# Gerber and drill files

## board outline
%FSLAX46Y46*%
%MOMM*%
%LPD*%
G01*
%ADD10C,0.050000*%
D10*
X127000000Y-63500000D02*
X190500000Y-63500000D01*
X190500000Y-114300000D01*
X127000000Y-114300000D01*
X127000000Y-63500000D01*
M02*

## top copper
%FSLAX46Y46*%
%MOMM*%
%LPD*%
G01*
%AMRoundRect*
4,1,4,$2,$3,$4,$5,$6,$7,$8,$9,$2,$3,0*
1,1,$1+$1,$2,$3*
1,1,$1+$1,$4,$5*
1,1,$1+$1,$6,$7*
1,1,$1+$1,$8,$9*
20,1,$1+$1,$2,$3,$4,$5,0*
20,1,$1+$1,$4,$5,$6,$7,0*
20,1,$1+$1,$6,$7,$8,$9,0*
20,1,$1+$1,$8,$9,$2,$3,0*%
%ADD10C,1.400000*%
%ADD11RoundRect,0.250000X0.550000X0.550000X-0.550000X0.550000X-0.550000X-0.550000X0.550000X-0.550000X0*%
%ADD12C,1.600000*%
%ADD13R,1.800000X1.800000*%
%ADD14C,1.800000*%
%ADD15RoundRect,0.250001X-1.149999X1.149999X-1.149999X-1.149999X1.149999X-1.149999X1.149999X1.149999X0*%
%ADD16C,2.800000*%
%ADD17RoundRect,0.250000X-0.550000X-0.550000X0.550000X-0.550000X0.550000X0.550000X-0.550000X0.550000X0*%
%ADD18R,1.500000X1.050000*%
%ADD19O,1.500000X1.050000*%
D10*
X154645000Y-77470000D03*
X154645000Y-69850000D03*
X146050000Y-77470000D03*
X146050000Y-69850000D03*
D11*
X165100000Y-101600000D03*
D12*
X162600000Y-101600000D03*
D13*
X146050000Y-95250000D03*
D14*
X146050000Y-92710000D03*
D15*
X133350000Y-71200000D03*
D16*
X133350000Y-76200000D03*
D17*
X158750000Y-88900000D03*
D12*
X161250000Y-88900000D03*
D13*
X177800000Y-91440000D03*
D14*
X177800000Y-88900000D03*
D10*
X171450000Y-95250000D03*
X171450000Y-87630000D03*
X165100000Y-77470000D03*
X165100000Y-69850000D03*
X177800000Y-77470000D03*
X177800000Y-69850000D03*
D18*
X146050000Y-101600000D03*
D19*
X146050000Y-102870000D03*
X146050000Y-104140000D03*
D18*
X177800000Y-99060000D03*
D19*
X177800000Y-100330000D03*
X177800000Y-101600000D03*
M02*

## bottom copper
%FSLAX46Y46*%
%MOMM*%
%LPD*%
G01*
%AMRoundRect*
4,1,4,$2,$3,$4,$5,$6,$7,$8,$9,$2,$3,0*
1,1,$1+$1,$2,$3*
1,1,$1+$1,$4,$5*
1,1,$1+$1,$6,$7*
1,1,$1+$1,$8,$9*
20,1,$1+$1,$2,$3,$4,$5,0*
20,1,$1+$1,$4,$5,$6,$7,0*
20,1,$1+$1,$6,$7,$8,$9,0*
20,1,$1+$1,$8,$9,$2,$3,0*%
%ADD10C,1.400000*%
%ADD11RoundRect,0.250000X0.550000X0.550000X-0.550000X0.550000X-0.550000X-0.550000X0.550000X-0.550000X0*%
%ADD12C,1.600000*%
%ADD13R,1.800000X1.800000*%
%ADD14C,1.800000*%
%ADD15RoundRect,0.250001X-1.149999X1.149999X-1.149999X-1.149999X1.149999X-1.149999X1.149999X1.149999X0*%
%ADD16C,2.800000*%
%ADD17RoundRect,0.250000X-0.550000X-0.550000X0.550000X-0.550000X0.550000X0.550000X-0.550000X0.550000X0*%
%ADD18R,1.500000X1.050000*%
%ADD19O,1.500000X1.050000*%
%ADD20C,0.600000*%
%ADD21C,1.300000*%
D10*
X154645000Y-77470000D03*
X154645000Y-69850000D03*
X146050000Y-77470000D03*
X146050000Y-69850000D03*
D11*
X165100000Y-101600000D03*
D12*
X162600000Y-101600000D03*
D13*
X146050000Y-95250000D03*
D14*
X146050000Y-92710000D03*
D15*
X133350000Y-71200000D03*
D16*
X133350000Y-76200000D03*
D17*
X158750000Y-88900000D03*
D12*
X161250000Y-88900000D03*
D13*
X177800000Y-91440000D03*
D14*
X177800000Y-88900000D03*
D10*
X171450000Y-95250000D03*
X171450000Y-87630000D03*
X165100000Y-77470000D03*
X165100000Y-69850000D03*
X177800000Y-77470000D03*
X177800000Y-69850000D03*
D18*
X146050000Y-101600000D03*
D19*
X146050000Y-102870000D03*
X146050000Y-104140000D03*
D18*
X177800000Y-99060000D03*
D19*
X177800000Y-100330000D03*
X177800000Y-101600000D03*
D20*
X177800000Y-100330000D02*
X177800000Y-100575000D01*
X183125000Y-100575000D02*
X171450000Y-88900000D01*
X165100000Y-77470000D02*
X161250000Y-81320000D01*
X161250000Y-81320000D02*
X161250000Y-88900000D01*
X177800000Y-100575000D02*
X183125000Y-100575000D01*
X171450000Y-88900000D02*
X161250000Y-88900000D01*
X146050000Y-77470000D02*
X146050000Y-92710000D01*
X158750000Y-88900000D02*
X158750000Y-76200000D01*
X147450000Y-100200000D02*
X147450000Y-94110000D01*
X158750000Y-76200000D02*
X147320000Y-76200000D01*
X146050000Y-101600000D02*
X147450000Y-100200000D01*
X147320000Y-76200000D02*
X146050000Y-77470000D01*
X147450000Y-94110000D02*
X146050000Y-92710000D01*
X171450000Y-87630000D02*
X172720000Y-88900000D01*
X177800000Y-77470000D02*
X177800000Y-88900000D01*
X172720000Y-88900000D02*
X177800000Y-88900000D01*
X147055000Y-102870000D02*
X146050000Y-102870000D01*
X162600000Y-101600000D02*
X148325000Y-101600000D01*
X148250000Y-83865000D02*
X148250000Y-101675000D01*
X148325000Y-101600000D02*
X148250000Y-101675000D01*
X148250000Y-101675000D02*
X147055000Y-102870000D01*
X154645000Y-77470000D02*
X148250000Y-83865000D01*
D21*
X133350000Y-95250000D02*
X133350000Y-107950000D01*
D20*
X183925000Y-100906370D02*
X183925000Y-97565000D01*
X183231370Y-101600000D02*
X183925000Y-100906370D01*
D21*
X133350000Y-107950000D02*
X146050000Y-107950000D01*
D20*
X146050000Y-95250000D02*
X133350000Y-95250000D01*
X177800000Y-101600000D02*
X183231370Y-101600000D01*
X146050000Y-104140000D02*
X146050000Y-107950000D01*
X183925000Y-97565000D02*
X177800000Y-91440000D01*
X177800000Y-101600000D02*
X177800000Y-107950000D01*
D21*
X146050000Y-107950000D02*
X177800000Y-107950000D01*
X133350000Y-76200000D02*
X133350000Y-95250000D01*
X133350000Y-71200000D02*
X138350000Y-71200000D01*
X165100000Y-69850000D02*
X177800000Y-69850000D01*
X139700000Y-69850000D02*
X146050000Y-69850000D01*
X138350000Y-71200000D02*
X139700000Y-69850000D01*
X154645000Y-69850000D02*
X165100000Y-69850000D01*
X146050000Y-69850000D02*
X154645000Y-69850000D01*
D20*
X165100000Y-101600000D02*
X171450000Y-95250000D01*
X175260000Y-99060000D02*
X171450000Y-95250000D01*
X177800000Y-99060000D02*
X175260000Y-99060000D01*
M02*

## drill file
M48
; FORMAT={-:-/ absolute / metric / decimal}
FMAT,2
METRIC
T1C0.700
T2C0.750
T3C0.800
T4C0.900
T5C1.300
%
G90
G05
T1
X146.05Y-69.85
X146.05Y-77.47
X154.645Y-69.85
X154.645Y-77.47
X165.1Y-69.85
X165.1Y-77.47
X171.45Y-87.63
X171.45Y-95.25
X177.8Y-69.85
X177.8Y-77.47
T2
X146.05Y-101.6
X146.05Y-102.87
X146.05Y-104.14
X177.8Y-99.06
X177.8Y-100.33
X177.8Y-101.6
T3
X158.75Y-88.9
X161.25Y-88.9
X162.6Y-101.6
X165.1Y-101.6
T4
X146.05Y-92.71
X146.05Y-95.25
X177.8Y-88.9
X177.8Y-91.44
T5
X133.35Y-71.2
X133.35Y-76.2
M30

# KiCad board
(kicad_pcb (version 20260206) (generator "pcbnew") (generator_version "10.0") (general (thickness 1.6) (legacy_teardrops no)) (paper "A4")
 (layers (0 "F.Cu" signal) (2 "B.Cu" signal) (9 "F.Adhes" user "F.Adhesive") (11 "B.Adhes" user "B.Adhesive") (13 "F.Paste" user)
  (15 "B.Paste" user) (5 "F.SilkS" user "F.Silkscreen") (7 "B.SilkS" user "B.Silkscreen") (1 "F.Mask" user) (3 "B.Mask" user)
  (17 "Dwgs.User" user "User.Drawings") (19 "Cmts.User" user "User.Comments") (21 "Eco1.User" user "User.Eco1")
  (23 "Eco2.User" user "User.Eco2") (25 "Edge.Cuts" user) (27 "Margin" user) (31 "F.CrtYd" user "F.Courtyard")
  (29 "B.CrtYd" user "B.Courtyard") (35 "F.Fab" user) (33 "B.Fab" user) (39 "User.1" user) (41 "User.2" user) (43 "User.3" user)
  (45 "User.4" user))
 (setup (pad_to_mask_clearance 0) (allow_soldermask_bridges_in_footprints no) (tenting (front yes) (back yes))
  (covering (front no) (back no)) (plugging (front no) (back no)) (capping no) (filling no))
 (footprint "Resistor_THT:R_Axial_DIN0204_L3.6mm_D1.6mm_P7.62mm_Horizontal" (layer "F.Cu") (at 154.645 77.47 90)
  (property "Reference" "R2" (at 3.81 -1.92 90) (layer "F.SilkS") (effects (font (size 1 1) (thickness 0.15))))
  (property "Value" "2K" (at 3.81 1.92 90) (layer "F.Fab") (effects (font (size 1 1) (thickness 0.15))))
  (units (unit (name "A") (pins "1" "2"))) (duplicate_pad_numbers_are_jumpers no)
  (pad "1" thru_hole circle (at 0 0 90) (size 1.4 1.4) (drill 0.7) (layers "*.Cu" "*.Mask") (remove_unused_layers no) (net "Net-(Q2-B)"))
  (pad "2" thru_hole circle (at 7.62 0 90) (size 1.4 1.4) (drill 0.7) (layers "*.Cu" "*.Mask") (remove_unused_layers no) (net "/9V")))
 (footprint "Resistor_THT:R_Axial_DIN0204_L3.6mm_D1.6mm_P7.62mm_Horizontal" (layer "F.Cu") (at 146.05 77.47 90)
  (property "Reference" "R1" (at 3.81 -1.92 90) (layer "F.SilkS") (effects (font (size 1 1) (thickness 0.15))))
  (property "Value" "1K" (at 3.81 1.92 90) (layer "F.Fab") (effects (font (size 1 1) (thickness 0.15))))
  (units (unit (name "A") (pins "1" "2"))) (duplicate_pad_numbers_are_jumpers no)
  (pad "1" thru_hole circle (at 0 0 90) (size 1.4 1.4) (drill 0.7) (layers "*.Cu" "*.Mask") (remove_unused_layers no) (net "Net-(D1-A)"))
  (pad "2" thru_hole circle (at 7.62 0 90) (size 1.4 1.4) (drill 0.7) (layers "*.Cu" "*.Mask") (remove_unused_layers no) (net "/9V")))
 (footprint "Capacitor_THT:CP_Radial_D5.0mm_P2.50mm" (layer "F.Cu") (at 165.1 101.6 180)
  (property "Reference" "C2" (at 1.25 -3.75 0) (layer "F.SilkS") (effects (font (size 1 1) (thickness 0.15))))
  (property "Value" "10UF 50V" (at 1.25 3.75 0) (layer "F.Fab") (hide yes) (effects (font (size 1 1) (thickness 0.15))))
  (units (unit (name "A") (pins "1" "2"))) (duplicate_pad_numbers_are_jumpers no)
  (pad "1" thru_hole roundrect (at 0 0 180) (size 1.6 1.6) (drill 0.8) (layers "*.Cu" "*.Mask") (remove_unused_layers no)
   (roundrect_rratio 0.15625) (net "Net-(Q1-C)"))
  (pad "2" thru_hole circle (at 2.5 0 180) (size 1.6 1.6) (drill 0.8) (layers "*.Cu" "*.Mask") (remove_unused_layers no) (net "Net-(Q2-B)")))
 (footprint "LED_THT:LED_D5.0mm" (layer "F.Cu") (at 146.05 95.25 90)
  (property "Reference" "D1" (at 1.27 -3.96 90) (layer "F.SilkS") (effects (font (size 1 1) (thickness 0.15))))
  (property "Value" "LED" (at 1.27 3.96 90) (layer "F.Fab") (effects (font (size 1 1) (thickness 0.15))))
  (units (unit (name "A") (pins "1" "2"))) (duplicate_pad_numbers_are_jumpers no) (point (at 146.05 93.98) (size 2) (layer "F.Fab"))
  (pad "1" thru_hole rect (at 0 0 90) (size 1.8 1.8) (drill 0.9) (layers "*.Cu" "*.Mask") (remove_unused_layers no) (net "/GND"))
  (pad "2" thru_hole circle (at 2.54 0 90) (size 1.8 1.8) (drill 0.9) (layers "*.Cu" "*.Mask") (remove_unused_layers no) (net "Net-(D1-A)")))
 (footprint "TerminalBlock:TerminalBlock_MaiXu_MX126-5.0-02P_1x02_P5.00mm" (layer "F.Cu") (at 133.35 71.2 -90)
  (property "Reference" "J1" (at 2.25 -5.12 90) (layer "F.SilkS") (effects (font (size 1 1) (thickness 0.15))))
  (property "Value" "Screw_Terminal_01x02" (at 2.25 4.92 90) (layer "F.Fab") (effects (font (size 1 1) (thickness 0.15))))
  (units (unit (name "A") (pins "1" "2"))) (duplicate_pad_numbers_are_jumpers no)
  (pad "1" thru_hole roundrect (at 0 0 270) (size 2.8 2.8) (drill 1.3) (layers "*.Cu" "*.Mask") (remove_unused_layers no)
   (roundrect_rratio 0.089286) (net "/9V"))
  (pad "2" thru_hole circle (at 5 0 270) (size 2.8 2.8) (drill 1.3) (layers "*.Cu" "*.Mask") (remove_unused_layers no) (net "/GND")))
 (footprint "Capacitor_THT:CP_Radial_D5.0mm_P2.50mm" (layer "F.Cu") (at 158.75 88.9)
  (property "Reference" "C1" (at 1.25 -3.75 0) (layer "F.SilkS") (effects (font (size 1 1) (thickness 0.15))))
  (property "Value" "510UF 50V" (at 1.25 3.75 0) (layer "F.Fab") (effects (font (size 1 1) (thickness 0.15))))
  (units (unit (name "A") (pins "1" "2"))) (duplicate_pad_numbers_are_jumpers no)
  (pad "1" thru_hole roundrect (at 0 0) (size 1.6 1.6) (drill 0.8) (layers "*.Cu" "*.Mask") (remove_unused_layers no)
   (roundrect_rratio 0.15625) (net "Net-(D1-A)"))
  (pad "2" thru_hole circle (at 2.5 0) (size 1.6 1.6) (drill 0.8) (layers "*.Cu" "*.Mask") (remove_unused_layers no) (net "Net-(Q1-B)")))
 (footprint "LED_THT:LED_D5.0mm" (layer "F.Cu") (at 177.8 91.44 90)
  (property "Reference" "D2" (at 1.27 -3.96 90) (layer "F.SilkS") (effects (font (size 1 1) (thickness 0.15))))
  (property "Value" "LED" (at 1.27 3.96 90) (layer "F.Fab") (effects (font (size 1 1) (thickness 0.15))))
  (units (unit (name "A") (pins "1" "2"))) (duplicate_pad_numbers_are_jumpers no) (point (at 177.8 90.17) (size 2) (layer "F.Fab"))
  (pad "1" thru_hole rect (at 0 0 90) (size 1.8 1.8) (drill 0.9) (layers "*.Cu" "*.Mask") (remove_unused_layers no) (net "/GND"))
  (pad "2" thru_hole circle (at 2.54 0 90) (size 1.8 1.8) (drill 0.9) (layers "*.Cu" "*.Mask") (remove_unused_layers no) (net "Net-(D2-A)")))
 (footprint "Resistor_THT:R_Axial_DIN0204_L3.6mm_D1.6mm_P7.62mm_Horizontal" (layer "F.Cu") (at 171.45 95.25 90)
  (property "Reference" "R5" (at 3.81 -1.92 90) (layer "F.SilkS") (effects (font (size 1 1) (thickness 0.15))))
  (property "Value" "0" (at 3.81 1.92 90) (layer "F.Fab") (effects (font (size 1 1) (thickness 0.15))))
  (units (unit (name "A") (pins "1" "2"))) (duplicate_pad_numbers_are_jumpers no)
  (pad "1" thru_hole circle (at 0 0 90) (size 1.4 1.4) (drill 0.7) (layers "*.Cu" "*.Mask") (remove_unused_layers no) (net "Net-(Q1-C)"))
  (pad "2" thru_hole circle (at 7.62 0 90) (size 1.4 1.4) (drill 0.7) (layers "*.Cu" "*.Mask") (remove_unused_layers no) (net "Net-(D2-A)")))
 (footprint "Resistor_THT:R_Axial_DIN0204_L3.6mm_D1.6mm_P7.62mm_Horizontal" (layer "F.Cu") (at 165.1 77.47 90)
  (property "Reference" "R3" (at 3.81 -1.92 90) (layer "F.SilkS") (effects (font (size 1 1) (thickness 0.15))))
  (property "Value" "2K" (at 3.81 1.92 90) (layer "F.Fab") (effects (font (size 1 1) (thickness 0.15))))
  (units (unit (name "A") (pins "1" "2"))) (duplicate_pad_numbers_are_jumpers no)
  (pad "1" thru_hole circle (at 0 0 90) (size 1.4 1.4) (drill 0.7) (layers "*.Cu" "*.Mask") (remove_unused_layers no) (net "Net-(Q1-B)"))
  (pad "2" thru_hole circle (at 7.62 0 90) (size 1.4 1.4) (drill 0.7) (layers "*.Cu" "*.Mask") (remove_unused_layers no) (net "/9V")))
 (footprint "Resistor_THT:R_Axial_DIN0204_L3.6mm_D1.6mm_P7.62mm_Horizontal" (layer "F.Cu") (at 177.8 77.47 90)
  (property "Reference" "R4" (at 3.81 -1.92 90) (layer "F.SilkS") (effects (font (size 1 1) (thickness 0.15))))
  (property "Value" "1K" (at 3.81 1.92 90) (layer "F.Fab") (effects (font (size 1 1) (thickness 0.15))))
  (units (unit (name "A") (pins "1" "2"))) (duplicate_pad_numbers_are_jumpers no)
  (pad "1" thru_hole circle (at 0 0 90) (size 1.4 1.4) (drill 0.7) (layers "*.Cu" "*.Mask") (remove_unused_layers no) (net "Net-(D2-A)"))
  (pad "2" thru_hole circle (at 7.62 0 90) (size 1.4 1.4) (drill 0.7) (layers "*.Cu" "*.Mask") (remove_unused_layers no) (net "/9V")))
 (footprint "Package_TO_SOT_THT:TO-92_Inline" (layer "F.Cu") (at 146.05 101.6 -90)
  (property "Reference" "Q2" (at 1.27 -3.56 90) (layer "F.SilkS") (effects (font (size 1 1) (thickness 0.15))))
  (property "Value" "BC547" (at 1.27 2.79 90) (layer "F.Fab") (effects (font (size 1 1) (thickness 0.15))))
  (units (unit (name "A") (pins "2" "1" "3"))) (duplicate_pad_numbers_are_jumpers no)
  (pad "1" thru_hole rect (at 0 0 270) (size 1.05 1.5) (drill 0.75) (layers "*.Cu" "*.Mask") (remove_unused_layers no) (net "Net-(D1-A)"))
  (pad "2" thru_hole oval (at 1.27 0 270) (size 1.05 1.5) (drill 0.75) (layers "*.Cu" "*.Mask") (remove_unused_layers no) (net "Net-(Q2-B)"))
  (pad "3" thru_hole oval (at 2.54 0 270) (size 1.05 1.5) (drill 0.75) (layers "*.Cu" "*.Mask") (remove_unused_layers no) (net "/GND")))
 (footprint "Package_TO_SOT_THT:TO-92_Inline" (layer "F.Cu") (at 177.8 99.06 -90)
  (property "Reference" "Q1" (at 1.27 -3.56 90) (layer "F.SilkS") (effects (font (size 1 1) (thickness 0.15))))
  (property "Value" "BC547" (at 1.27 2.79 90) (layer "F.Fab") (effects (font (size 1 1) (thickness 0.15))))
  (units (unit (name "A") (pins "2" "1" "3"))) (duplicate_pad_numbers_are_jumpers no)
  (pad "1" thru_hole rect (at 0 0 270) (size 1.05 1.5) (drill 0.75) (layers "*.Cu" "*.Mask") (remove_unused_layers no) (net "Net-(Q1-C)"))
  (pad "2" thru_hole oval (at 1.27 0 270) (size 1.05 1.5) (drill 0.75) (layers "*.Cu" "*.Mask") (remove_unused_layers no) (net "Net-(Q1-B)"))
  (pad "3" thru_hole oval (at 2.54 0 270) (size 1.05 1.5) (drill 0.75) (layers "*.Cu" "*.Mask") (remove_unused_layers no) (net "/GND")))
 (gr_rect (start 127 63.5) (end 190.5 114.3) (stroke (width 0.05) (type default)) (fill no) (layer "Edge.Cuts"))
 (segment (start 177.8 100.33) (end 177.8 100.575) (width 0.6) (layer "B.Cu") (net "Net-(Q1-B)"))
 (segment (start 183.125 100.575) (end 171.45 88.9) (width 0.6) (layer "B.Cu") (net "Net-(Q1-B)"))
 (segment (start 165.1 77.47) (end 161.25 81.32) (width 0.6) (layer "B.Cu") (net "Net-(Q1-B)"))
 (segment (start 161.25 81.32) (end 161.25 88.9) (width 0.6) (layer "B.Cu") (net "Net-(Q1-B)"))
 (segment (start 177.8 100.575) (end 183.125 100.575) (width 0.6) (layer "B.Cu") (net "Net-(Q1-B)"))
 (segment (start 171.45 88.9) (end 161.25 88.9) (width 0.6) (layer "B.Cu") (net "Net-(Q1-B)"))
 (segment (start 146.05 77.47) (end 146.05 92.71) (width 0.6) (layer "B.Cu") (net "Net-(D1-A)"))
 (segment (start 158.75 88.9) (end 158.75 76.2) (width 0.6) (layer "B.Cu") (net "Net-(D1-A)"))
 (segment (start 147.45 100.2) (end 147.45 94.11) (width 0.6) (layer "B.Cu") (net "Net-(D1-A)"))
 (segment (start 158.75 76.2) (end 147.32 76.2) (width 0.6) (layer "B.Cu") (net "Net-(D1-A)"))
 (segment (start 146.05 101.6) (end 147.45 100.2) (width 0.6) (layer "B.Cu") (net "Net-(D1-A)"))
 (segment (start 147.32 76.2) (end 146.05 77.47) (width 0.6) (layer "B.Cu") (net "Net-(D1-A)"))
 (segment (start 147.45 94.11) (end 146.05 92.71) (width 0.6) (layer "B.Cu") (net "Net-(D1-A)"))
 (segment (start 171.45 87.63) (end 172.72 88.9) (width 0.6) (layer "B.Cu") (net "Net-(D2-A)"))
 (segment (start 177.8 77.47) (end 177.8 88.9) (width 0.6) (layer "B.Cu") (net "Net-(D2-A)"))
 (segment (start 172.72 88.9) (end 177.8 88.9) (width 0.6) (layer "B.Cu") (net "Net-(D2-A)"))
 (segment (start 147.055 102.87) (end 146.05 102.87) (width 0.6) (layer "B.Cu") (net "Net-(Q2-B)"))
 (segment (start 162.6 101.6) (end 148.325 101.6) (width 0.6) (layer "B.Cu") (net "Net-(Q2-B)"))
 (segment (start 148.25 83.865) (end 148.25 101.675) (width 0.6) (layer "B.Cu") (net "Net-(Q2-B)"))
 (segment (start 148.325 101.6) (end 148.25 101.675) (width 0.6) (layer "B.Cu") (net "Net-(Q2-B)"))
 (segment (start 148.25 101.675) (end 147.055 102.87) (width 0.6) (layer "B.Cu") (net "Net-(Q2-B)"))
 (segment (start 154.645 77.47) (end 148.25 83.865) (width 0.6) (layer "B.Cu") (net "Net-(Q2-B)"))
 (segment (start 133.35 95.25) (end 133.35 107.95) (width 1.3) (layer "B.Cu") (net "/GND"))
 (segment (start 183.925 100.90637) (end 183.925 97.565) (width 0.6) (layer "B.Cu") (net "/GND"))
 (segment (start 183.23137 101.6) (end 183.925 100.90637) (width 0.6) (layer "B.Cu") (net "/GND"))
 (segment (start 133.35 107.95) (end 146.05 107.95) (width 1.3) (layer "B.Cu") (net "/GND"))
 (segment (start 146.05 95.25) (end 133.35 95.25) (width 0.6) (layer "B.Cu") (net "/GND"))
 (segment (start 177.8 101.6) (end 183.23137 101.6) (width 0.6) (layer "B.Cu") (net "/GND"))
 (segment (start 146.05 104.14) (end 146.05 107.95) (width 0.6) (layer "B.Cu") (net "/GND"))
 (segment (start 183.925 97.565) (end 177.8 91.44) (width 0.6) (layer "B.Cu") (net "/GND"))
 (segment (start 177.8 101.6) (end 177.8 107.95) (width 0.6) (layer "B.Cu") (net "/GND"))
 (segment (start 146.05 107.95) (end 177.8 107.95) (width 1.3) (layer "B.Cu") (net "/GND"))
 (segment (start 133.35 76.2) (end 133.35 95.25) (width 1.3) (layer "B.Cu") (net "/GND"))
 (segment (start 133.35 71.2) (end 138.35 71.2) (width 1.3) (layer "B.Cu") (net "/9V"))
 (segment (start 165.1 69.85) (end 177.8 69.85) (width 1.3) (layer "B.Cu") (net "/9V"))
 (segment (start 139.7 69.85) (end 146.05 69.85) (width 1.3) (layer "B.Cu") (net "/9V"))
 (segment (start 138.35 71.2) (end 139.7 69.85) (width 1.3) (layer "B.Cu") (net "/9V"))
 (segment (start 154.645 69.85) (end 165.1 69.85) (width 1.3) (layer "B.Cu") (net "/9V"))
 (segment (start 146.05 69.85) (end 154.645 69.85) (width 1.3) (layer "B.Cu") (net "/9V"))
 (segment (start 165.1 101.6) (end 171.45 95.25) (width 0.6) (layer "B.Cu") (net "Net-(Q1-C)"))
 (segment (start 175.26 99.06) (end 171.45 95.25) (width 0.6) (layer "B.Cu") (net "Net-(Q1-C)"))
 (segment (start 177.8 99.06) (end 175.26 99.06) (width 0.6) (layer "B.Cu") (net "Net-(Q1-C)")))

